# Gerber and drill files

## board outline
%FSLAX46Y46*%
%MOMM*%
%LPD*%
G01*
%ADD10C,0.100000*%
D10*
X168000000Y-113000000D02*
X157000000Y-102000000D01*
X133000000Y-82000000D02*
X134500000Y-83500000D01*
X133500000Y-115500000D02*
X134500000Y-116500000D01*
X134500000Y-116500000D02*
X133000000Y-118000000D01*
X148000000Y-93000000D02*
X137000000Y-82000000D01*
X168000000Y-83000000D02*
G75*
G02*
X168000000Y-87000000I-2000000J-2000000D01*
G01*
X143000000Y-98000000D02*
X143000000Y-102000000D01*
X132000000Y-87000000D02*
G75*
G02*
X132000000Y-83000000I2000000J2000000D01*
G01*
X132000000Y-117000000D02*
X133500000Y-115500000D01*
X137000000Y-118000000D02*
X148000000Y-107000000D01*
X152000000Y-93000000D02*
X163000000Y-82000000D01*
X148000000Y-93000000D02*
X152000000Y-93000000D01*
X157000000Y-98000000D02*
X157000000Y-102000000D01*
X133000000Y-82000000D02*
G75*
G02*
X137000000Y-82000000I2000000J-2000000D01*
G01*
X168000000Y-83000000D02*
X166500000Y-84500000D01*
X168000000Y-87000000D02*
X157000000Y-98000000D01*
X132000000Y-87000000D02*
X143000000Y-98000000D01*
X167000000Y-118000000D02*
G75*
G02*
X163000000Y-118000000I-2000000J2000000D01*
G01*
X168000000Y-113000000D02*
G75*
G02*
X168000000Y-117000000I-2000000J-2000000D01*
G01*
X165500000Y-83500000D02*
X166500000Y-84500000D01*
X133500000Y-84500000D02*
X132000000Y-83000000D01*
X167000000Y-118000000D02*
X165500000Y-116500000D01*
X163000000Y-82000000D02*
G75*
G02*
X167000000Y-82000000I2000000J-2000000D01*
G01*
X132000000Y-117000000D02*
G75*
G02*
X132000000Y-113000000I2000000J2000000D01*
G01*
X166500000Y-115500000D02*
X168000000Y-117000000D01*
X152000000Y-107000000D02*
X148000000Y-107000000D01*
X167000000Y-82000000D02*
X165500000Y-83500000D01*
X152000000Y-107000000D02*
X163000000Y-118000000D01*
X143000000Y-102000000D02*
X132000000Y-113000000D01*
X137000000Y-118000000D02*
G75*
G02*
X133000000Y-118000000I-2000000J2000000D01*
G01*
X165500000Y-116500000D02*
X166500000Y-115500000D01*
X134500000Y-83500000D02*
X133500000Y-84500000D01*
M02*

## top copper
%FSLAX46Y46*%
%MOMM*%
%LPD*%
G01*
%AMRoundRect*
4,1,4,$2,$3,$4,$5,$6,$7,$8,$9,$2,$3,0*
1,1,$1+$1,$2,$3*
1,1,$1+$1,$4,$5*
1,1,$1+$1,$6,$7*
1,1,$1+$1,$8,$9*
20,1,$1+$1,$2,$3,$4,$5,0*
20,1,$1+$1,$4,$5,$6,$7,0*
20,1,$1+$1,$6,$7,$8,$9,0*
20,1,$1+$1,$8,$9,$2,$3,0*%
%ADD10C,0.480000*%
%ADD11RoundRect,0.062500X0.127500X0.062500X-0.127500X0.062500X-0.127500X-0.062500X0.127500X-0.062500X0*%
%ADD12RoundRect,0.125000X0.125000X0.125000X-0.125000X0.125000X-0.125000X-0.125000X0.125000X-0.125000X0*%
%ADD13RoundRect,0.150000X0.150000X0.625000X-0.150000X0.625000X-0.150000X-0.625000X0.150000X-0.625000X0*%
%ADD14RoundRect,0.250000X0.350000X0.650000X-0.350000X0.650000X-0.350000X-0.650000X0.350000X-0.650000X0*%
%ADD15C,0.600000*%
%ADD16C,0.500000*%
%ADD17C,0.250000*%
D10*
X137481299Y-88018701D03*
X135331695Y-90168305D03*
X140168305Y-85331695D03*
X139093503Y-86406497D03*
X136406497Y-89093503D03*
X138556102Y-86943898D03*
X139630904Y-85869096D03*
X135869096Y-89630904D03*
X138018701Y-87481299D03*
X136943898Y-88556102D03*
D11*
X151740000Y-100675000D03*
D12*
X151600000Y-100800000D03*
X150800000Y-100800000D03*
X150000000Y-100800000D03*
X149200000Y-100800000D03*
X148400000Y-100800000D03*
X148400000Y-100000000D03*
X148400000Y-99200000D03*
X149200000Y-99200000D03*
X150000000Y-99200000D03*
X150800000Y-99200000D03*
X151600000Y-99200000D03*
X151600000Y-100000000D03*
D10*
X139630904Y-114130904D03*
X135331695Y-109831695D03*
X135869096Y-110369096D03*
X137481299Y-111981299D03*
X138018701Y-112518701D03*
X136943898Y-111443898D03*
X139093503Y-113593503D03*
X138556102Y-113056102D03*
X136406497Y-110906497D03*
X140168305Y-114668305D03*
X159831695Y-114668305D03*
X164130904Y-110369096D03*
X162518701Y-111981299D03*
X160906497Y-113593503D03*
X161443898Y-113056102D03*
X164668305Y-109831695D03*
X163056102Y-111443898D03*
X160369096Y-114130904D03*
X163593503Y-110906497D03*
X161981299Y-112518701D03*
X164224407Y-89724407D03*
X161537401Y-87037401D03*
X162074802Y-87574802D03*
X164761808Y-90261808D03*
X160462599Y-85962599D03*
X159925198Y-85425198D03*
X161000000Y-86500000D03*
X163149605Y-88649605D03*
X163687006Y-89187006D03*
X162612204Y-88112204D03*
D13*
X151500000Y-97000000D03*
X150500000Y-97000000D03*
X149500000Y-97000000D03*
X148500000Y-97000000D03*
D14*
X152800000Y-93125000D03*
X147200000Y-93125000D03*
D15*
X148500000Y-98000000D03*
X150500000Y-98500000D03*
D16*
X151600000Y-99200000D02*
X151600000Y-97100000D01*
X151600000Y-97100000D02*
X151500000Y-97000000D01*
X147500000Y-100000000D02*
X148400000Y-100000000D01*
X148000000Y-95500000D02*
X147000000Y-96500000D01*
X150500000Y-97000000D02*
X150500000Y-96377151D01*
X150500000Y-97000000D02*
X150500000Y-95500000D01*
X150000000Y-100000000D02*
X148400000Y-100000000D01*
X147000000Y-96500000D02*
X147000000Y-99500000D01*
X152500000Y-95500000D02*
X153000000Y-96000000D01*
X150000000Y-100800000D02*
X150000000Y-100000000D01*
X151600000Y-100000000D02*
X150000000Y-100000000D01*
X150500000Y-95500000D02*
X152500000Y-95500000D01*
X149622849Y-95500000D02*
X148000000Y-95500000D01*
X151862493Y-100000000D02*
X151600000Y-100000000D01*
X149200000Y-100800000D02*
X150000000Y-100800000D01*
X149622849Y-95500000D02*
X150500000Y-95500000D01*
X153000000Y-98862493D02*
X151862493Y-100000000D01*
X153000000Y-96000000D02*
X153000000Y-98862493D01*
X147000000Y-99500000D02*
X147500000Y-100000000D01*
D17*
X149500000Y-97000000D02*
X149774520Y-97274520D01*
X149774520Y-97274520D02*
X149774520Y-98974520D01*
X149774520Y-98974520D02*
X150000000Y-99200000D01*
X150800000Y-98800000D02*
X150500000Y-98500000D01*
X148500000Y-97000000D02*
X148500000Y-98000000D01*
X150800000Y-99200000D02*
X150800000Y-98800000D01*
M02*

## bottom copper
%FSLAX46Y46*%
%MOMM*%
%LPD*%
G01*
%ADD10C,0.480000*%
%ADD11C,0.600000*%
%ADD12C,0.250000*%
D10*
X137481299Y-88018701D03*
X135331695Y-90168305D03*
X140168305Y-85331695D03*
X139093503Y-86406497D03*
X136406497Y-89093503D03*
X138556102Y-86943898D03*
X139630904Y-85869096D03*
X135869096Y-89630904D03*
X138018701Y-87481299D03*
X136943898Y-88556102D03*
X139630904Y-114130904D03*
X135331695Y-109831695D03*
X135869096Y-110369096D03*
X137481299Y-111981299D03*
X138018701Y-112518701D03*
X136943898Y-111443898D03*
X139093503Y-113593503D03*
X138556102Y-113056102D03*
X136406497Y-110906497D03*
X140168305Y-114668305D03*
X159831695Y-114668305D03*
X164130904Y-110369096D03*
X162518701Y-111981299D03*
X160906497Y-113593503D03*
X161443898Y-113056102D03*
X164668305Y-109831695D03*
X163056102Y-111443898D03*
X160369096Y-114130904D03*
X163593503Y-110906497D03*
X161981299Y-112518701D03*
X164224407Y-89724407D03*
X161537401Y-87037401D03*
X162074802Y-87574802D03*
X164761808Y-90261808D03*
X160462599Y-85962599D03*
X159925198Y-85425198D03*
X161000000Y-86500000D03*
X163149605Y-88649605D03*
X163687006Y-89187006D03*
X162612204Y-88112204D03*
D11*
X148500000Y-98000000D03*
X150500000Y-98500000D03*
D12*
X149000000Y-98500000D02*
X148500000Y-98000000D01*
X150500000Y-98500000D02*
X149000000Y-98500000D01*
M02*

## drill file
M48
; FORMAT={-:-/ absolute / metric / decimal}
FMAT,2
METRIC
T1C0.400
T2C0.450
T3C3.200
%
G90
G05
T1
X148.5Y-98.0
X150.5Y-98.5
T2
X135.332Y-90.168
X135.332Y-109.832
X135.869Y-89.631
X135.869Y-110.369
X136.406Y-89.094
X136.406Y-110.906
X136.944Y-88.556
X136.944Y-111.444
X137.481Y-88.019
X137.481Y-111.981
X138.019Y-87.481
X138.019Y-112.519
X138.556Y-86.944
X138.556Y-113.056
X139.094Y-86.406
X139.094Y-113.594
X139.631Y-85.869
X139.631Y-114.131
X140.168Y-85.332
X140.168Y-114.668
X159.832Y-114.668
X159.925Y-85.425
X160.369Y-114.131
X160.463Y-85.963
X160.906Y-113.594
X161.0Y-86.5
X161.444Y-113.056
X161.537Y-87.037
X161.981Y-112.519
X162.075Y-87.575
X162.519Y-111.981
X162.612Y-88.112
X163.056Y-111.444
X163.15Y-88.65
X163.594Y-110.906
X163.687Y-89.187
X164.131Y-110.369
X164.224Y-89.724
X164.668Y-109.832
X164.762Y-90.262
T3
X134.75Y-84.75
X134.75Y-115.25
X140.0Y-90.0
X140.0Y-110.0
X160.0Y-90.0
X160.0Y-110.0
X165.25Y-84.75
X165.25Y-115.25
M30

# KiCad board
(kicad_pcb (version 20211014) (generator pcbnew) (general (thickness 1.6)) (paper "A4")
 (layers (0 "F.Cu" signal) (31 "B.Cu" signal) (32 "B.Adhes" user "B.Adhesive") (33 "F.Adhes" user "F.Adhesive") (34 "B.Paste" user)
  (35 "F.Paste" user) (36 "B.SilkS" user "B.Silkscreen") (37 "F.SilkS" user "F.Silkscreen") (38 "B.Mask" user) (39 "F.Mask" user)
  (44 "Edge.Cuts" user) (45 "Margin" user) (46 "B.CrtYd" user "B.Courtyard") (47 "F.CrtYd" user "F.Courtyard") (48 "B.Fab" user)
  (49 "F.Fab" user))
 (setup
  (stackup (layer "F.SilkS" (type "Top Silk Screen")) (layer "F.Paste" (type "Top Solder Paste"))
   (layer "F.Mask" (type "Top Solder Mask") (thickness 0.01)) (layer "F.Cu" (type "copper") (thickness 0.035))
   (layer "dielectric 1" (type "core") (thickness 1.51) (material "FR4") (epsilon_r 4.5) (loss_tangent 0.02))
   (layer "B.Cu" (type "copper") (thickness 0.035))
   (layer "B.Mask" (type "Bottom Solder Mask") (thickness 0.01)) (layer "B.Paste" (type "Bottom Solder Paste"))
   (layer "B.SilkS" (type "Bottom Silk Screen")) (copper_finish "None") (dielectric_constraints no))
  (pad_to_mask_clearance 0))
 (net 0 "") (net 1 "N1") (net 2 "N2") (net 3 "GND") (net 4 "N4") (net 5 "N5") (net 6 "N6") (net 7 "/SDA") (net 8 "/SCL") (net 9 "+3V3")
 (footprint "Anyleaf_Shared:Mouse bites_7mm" (layer "F.Cu") (at 137.75 87.75 45)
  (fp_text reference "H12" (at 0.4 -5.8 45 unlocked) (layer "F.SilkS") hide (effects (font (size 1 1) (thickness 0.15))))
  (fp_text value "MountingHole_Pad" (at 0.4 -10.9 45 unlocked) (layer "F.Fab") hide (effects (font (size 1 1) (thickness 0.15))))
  (pad "" np_thru_hole circle (at -0.38 0 45) (size 0.48 0.48) (drill 0.45) (layers F&B.Cu *.Mask))
  (pad "" np_thru_hole circle (at -3.42 0 45) (size 0.48 0.48) (drill 0.45) (layers F&B.Cu *.Mask))
  (pad "" np_thru_hole circle (at 3.42 0 45) (size 0.48 0.48) (drill 0.45) (layers F&B.Cu *.Mask))
  (pad "" np_thru_hole circle (at 1.9 0 45) (size 0.48 0.48) (drill 0.45) (layers F&B.Cu *.Mask))
  (pad "" np_thru_hole circle (at -1.9 0 45) (size 0.48 0.48) (drill 0.45) (layers F&B.Cu *.Mask))
  (pad "" np_thru_hole circle (at 1.14 0 45) (size 0.48 0.48) (drill 0.45) (layers F&B.Cu *.Mask))
  (pad "" np_thru_hole circle (at 2.66 0 45) (size 0.48 0.48) (drill 0.45) (layers F&B.Cu *.Mask))
  (pad "" np_thru_hole circle (at -2.66 0 45) (size 0.48 0.48) (drill 0.45) (layers F&B.Cu *.Mask))
  (pad "" np_thru_hole circle (at 0.38 0 45) (size 0.48 0.48) (drill 0.45) (layers F&B.Cu *.Mask))
  (pad "" np_thru_hole circle (at -1.14 0 45) (size 0.48 0.48) (drill 0.45) (layers F&B.Cu *.Mask)))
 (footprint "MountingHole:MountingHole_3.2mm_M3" (layer "F.Cu") (at 134.75 115.25)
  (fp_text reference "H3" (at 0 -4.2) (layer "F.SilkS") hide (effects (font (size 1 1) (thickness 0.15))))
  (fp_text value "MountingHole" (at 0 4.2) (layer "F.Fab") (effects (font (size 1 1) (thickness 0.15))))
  (pad "" np_thru_hole circle locked (at 0 0) (size 3.2 3.2) (drill 3.2) (layers *.Cu *.Mask)))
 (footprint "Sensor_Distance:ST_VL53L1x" (layer "F.Cu") (at 150 100 180)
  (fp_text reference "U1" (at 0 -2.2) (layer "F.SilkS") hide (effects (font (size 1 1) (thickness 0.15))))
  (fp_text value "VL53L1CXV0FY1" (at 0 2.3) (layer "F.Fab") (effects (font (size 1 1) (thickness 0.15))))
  (pad "1" smd roundrect locked (at -1.74 -0.675 180) (size 0.38 0.25) (layers "F.Cu" "F.Paste" "F.Mask") (roundrect_rratio 0.25)
   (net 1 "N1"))
  (pad "1" smd roundrect locked (at -1.6 -0.8 180) (size 0.5 0.5) (layers "F.Cu" "F.Paste" "F.Mask") (roundrect_rratio 0.25) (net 1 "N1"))
  (pad "2" smd roundrect locked (at -0.8 -0.8 180) (size 0.5 0.5) (layers "F.Cu" "F.Paste" "F.Mask") (roundrect_rratio 0.25) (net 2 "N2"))
  (pad "3" smd roundrect locked (at 0 -0.8 180) (size 0.5 0.5) (layers "F.Cu" "F.Paste" "F.Mask") (roundrect_rratio 0.25) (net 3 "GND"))
  (pad "4" smd roundrect locked (at 0.8 -0.8 180) (size 0.5 0.5) (layers "F.Cu" "F.Paste" "F.Mask") (roundrect_rratio 0.25) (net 3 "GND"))
  (pad "5" smd roundrect locked (at 1.6 -0.8 180) (size 0.5 0.5) (layers "F.Cu" "F.Paste" "F.Mask") (roundrect_rratio 0.25) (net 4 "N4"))
  (pad "6" smd roundrect locked (at 1.6 0 180) (size 0.5 0.5) (layers "F.Cu" "F.Paste" "F.Mask") (roundrect_rratio 0.25) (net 3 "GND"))
  (pad "7" smd roundrect locked (at 1.6 0.8 180) (size 0.5 0.5) (layers "F.Cu" "F.Paste" "F.Mask") (roundrect_rratio 0.25) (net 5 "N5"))
  (pad "8" smd roundrect locked (at 0.8 0.8 180) (size 0.5 0.5) (layers "F.Cu" "F.Paste" "F.Mask") (roundrect_rratio 0.25) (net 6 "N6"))
  (pad "9" smd roundrect locked (at 0 0.8 180) (size 0.5 0.5) (layers "F.Cu" "F.Paste" "F.Mask") (roundrect_rratio 0.25) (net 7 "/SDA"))
  (pad "10" smd roundrect locked (at -0.8 0.8 180) (size 0.5 0.5) (layers "F.Cu" "F.Paste" "F.Mask") (roundrect_rratio 0.25) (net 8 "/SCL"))
  (pad "11" smd roundrect locked (at -1.6 0.8 180) (size 0.5 0.5) (layers "F.Cu" "F.Paste" "F.Mask") (roundrect_rratio 0.25) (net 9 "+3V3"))
  (pad "12" smd roundrect locked (at -1.6 0 180) (size 0.5 0.5) (layers "F.Cu" "F.Paste" "F.Mask") (roundrect_rratio 0.25) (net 3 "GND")))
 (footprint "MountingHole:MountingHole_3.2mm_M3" (layer "F.Cu") (at 134.75 84.75)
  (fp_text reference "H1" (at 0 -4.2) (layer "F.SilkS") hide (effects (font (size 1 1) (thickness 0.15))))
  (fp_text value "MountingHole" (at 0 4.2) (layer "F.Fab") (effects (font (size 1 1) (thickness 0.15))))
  (pad "" np_thru_hole circle locked (at 0 0) (size 3.2 3.2) (drill 3.2) (layers *.Cu *.Mask)))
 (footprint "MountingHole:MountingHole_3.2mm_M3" (layer "F.Cu") (at 140 90)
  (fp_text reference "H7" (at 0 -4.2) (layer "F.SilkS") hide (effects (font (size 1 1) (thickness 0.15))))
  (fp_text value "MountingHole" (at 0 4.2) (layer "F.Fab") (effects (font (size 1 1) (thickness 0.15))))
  (pad "" np_thru_hole circle locked (at 0 0) (size 3.2 3.2) (drill 3.2) (layers *.Cu *.Mask)))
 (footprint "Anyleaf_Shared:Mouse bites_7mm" (layer "F.Cu") (at 137.75 112.25 135)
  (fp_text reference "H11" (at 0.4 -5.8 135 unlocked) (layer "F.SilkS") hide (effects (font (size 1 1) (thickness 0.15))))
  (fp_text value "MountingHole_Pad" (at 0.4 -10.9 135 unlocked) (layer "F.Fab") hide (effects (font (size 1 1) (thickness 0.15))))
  (pad "" np_thru_hole circle (at -2.66 0 135) (size 0.48 0.48) (drill 0.45) (layers F&B.Cu *.Mask))
  (pad "" np_thru_hole circle (at 3.42 0 135) (size 0.48 0.48) (drill 0.45) (layers F&B.Cu *.Mask))
  (pad "" np_thru_hole circle (at 2.66 0 135) (size 0.48 0.48) (drill 0.45) (layers F&B.Cu *.Mask))
  (pad "" np_thru_hole circle (at 0.38 0 135) (size 0.48 0.48) (drill 0.45) (layers F&B.Cu *.Mask))
  (pad "" np_thru_hole circle (at -0.38 0 135) (size 0.48 0.48) (drill 0.45) (layers F&B.Cu *.Mask))
  (pad "" np_thru_hole circle (at 1.14 0 135) (size 0.48 0.48) (drill 0.45) (layers F&B.Cu *.Mask))
  (pad "" np_thru_hole circle (at -1.9 0 135) (size 0.48 0.48) (drill 0.45) (layers F&B.Cu *.Mask))
  (pad "" np_thru_hole circle (at -1.14 0 135) (size 0.48 0.48) (drill 0.45) (layers F&B.Cu *.Mask))
  (pad "" np_thru_hole circle (at 1.9 0 135) (size 0.48 0.48) (drill 0.45) (layers F&B.Cu *.Mask))
  (pad "" np_thru_hole circle (at -3.42 0 135) (size 0.48 0.48) (drill 0.45) (layers F&B.Cu *.Mask)))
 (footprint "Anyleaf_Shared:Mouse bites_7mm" (layer "F.Cu") (at 162.25 112.25 45)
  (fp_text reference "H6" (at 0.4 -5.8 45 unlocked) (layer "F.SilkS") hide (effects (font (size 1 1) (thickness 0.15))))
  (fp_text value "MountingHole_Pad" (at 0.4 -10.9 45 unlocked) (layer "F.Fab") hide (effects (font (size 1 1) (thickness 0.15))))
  (pad "" np_thru_hole circle (at -3.42 0 45) (size 0.48 0.48) (drill 0.45) (layers F&B.Cu *.Mask))
  (pad "" np_thru_hole circle (at 2.66 0 45) (size 0.48 0.48) (drill 0.45) (layers F&B.Cu *.Mask))
  (pad "" np_thru_hole circle (at 0.38 0 45) (size 0.48 0.48) (drill 0.45) (layers F&B.Cu *.Mask))
  (pad "" np_thru_hole circle (at -1.9 0 45) (size 0.48 0.48) (drill 0.45) (layers F&B.Cu *.Mask))
  (pad "" np_thru_hole circle (at -1.14 0 45) (size 0.48 0.48) (drill 0.45) (layers F&B.Cu *.Mask))
  (pad "" np_thru_hole circle (at 3.42 0 45) (size 0.48 0.48) (drill 0.45) (layers F&B.Cu *.Mask))
  (pad "" np_thru_hole circle (at 1.14 0 45) (size 0.48 0.48) (drill 0.45) (layers F&B.Cu *.Mask))
  (pad "" np_thru_hole circle (at -2.66 0 45) (size 0.48 0.48) (drill 0.45) (layers F&B.Cu *.Mask))
  (pad "" np_thru_hole circle (at 1.9 0 45) (size 0.48 0.48) (drill 0.45) (layers F&B.Cu *.Mask))
  (pad "" np_thru_hole circle (at -0.38 0 45) (size 0.48 0.48) (drill 0.45) (layers F&B.Cu *.Mask)))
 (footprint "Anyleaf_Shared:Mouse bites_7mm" (layer "F.Cu") (at 162.343503 87.843503 135)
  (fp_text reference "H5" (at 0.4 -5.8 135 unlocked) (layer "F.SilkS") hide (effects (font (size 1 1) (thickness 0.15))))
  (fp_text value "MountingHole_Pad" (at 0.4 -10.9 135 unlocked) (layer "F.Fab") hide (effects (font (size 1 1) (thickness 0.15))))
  (pad "" np_thru_hole circle (at -2.66 0 135) (size 0.48 0.48) (drill 0.45) (layers F&B.Cu *.Mask))
  (pad "" np_thru_hole circle (at 1.14 0 135) (size 0.48 0.48) (drill 0.45) (layers F&B.Cu *.Mask))
  (pad "" np_thru_hole circle (at 0.38 0 135) (size 0.48 0.48) (drill 0.45) (layers F&B.Cu *.Mask))
  (pad "" np_thru_hole circle (at -3.42 0 135) (size 0.48 0.48) (drill 0.45) (layers F&B.Cu *.Mask))
  (pad "" np_thru_hole circle (at 2.66 0 135) (size 0.48 0.48) (drill 0.45) (layers F&B.Cu *.Mask))
  (pad "" np_thru_hole circle (at 3.42 0 135) (size 0.48 0.48) (drill 0.45) (layers F&B.Cu *.Mask))
  (pad "" np_thru_hole circle (at 1.9 0 135) (size 0.48 0.48) (drill 0.45) (layers F&B.Cu *.Mask))
  (pad "" np_thru_hole circle (at -1.14 0 135) (size 0.48 0.48) (drill 0.45) (layers F&B.Cu *.Mask))
  (pad "" np_thru_hole circle (at -1.9 0 135) (size 0.48 0.48) (drill 0.45) (layers F&B.Cu *.Mask))
  (pad "" np_thru_hole circle (at -0.38 0 135) (size 0.48 0.48) (drill 0.45) (layers F&B.Cu *.Mask)))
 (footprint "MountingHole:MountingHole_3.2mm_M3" (layer "F.Cu") (at 160 90)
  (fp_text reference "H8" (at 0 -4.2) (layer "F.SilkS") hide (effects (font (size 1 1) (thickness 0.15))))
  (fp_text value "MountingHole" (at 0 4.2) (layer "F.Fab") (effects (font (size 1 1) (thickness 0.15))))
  (pad "" np_thru_hole circle locked (at 0 0) (size 3.2 3.2) (drill 3.2) (layers *.Cu *.Mask)))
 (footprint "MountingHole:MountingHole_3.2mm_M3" (layer "F.Cu") (at 160 110)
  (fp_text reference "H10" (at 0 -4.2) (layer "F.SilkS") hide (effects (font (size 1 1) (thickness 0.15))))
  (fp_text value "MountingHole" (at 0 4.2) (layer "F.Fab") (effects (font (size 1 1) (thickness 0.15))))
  (pad "" np_thru_hole circle locked (at 0 0) (size 3.2 3.2) (drill 3.2) (layers *.Cu *.Mask)))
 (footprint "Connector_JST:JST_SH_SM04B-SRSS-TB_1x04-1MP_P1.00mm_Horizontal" (layer "F.Cu") (at 150 95 180)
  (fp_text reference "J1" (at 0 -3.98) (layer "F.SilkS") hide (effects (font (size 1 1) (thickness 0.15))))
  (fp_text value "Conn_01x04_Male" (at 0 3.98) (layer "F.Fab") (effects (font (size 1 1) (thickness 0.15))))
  (pad "1" smd roundrect locked (at -1.5 -2 180) (size 0.6 1.55) (layers "F.Cu" "F.Paste" "F.Mask") (roundrect_rratio 0.25) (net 9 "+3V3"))
  (pad "2" smd roundrect locked (at -0.5 -2 180) (size 0.6 1.55) (layers "F.Cu" "F.Paste" "F.Mask") (roundrect_rratio 0.25) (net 3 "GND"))
  (pad "3" smd roundrect locked (at 0.5 -2 180) (size 0.6 1.55) (layers "F.Cu" "F.Paste" "F.Mask") (roundrect_rratio 0.25) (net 7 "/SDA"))
  (pad "4" smd roundrect locked (at 1.5 -2 180) (size 0.6 1.55) (layers "F.Cu" "F.Paste" "F.Mask") (roundrect_rratio 0.25) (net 8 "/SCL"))
  (pad "MP" smd roundrect locked (at -2.8 1.875 180) (size 1.2 1.8) (layers "F.Cu" "F.Paste" "F.Mask") (roundrect_rratio 0.2083333333))
  (pad "MP" smd roundrect locked (at 2.8 1.875 180) (size 1.2 1.8) (layers "F.Cu" "F.Paste" "F.Mask") (roundrect_rratio 0.2083333333)))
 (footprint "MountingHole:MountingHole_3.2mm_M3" (layer "F.Cu") (at 165.25 115.25)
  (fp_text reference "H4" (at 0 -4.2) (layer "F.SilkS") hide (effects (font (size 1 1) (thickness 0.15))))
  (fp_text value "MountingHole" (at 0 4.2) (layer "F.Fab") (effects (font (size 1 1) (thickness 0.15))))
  (pad "" np_thru_hole circle locked (at 0 0) (size 3.2 3.2) (drill 3.2) (layers *.Cu *.Mask)))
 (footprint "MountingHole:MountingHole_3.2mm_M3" (layer "F.Cu") (at 165.25 84.75)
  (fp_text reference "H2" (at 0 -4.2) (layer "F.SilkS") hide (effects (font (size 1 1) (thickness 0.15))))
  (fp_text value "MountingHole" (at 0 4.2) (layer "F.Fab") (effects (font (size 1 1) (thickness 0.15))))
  (pad "" np_thru_hole circle locked (at 0 0) (size 3.2 3.2) (drill 3.2) (layers *.Cu *.Mask)))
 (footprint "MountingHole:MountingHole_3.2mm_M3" (layer "F.Cu") (at 140 110)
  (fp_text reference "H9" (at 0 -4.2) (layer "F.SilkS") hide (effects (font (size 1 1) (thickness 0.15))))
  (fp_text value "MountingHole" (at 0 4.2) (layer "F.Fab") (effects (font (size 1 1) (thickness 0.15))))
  (pad "" np_thru_hole circle locked (at 0 0) (size 3.2 3.2) (drill 3.2) (layers *.Cu *.Mask)))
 (gr_line (start 168 113) (end 157 102) (layer "Edge.Cuts") (width 0.1))
 (gr_line (start 133 82) (end 134.5 83.5) (layer "Edge.Cuts") (width 0.1))
 (gr_line (start 133.5 115.5) (end 134.5 116.5) (layer "Edge.Cuts") (width 0.1))
 (gr_line (start 134.5 116.5) (end 133 118) (layer "Edge.Cuts") (width 0.1))
 (gr_line (start 148 93) (end 137 82) (layer "Edge.Cuts") (width 0.1))
 (gr_arc (start 168 83) (mid 168.828427 85) (end 168 87) (layer "Edge.Cuts") (width 0.1))
 (gr_line (start 143 98) (end 143 102) (layer "Edge.Cuts") (width 0.1))
 (gr_arc (start 132 87) (mid 131.171573 85) (end 132 83) (layer "Edge.Cuts") (width 0.1))
 (gr_line (start 132 117) (end 133.5 115.5) (layer "Edge.Cuts") (width 0.1))
 (gr_line (start 137 118) (end 148 107) (layer "Edge.Cuts") (width 0.1))
 (gr_line (start 152 93) (end 163 82) (layer "Edge.Cuts") (width 0.1))
 (gr_line (start 148 93) (end 152 93) (layer "Edge.Cuts") (width 0.1))
 (gr_line (start 157 98) (end 157 102) (layer "Edge.Cuts") (width 0.1))
 (gr_arc (start 133 82) (mid 135 81.171573) (end 137 82) (layer "Edge.Cuts") (width 0.1))
 (gr_line (start 168 83) (end 166.5 84.5) (layer "Edge.Cuts") (width 0.1))
 (gr_line (start 168 87) (end 157 98) (layer "Edge.Cuts") (width 0.1))
 (gr_line (start 132 87) (end 143 98) (layer "Edge.Cuts") (width 0.1))
 (gr_arc (start 167 118) (mid 165 118.828427) (end 163 118) (layer "Edge.Cuts") (width 0.1))
 (gr_arc (start 168 113) (mid 168.828427 115) (end 168 117) (layer "Edge.Cuts") (width 0.1))
 (gr_line (start 165.5 83.5) (end 166.5 84.5) (layer "Edge.Cuts") (width 0.1))
 (gr_line (start 133.5 84.5) (end 132 83) (layer "Edge.Cuts") (width 0.1))
 (gr_line (start 167 118) (end 165.5 116.5) (layer "Edge.Cuts") (width 0.1))
 (gr_arc (start 163 82) (mid 165 81.171573) (end 167 82) (layer "Edge.Cuts") (width 0.1))
 (gr_arc (start 132 117) (mid 131.171573 115) (end 132 113) (layer "Edge.Cuts") (width 0.1))
 (gr_line (start 166.5 115.5) (end 168 117) (layer "Edge.Cuts") (width 0.1))
 (gr_line (start 152 107) (end 148 107) (layer "Edge.Cuts") (width 0.1))
 (gr_line (start 167 82) (end 165.5 83.5) (layer "Edge.Cuts") (width 0.1))
 (gr_line (start 152 107) (end 163 118) (layer "Edge.Cuts") (width 0.1))
 (gr_line (start 143 102) (end 132 113) (layer "Edge.Cuts") (width 0.1))
 (gr_arc (start 137 118) (mid 135 118.828427) (end 133 118) (layer "Edge.Cuts") (width 0.1))
 (gr_line (start 165.5 116.5) (end 166.5 115.5) (layer "Edge.Cuts") (width 0.1))
 (gr_line (start 134.5 83.5) (end 133.5 84.5) (layer "Edge.Cuts") (width 0.1))
 (segment (start 151.6 99.2) (end 151.6 97.1) (width 0.5) (layer "F.Cu") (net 9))
 (segment (start 151.6 97.1) (end 151.5 97) (width 0.5) (layer "F.Cu") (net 9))
 (segment (start 147.5 100) (end 148.4 100) (width 0.5) (layer "F.Cu") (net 3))
 (segment (start 148 95.5) (end 147 96.5) (width 0.5) (layer "F.Cu") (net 3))
 (segment (start 150.5 97) (end 150.5 96.377151) (width 0.5) (layer "F.Cu") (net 3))
 (segment (start 150.5 97) (end 150.5 95.5) (width 0.5) (layer "F.Cu") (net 3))
 (segment (start 150 100) (end 148.4 100) (width 0.5) (layer "F.Cu") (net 3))
 (segment (start 147 96.5) (end 147 99.5) (width 0.5) (layer "F.Cu") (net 3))
 (segment (start 152.5 95.5) (end 153 96) (width 0.5) (layer "F.Cu") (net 3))
 (segment (start 150 100.8) (end 150 100) (width 0.5) (layer "F.Cu") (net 3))
 (segment (start 151.6 100) (end 150 100) (width 0.5) (layer "F.Cu") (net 3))
 (segment (start 150.5 95.5) (end 152.5 95.5) (width 0.5) (layer "F.Cu") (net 3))
 (segment (start 149.622849 95.5) (end 148 95.5) (width 0.5) (layer "F.Cu") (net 3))
 (segment (start 151.862493 100) (end 151.6 100) (width 0.5) (layer "F.Cu") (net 3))
 (segment (start 149.2 100.8) (end 150 100.8) (width 0.5) (layer "F.Cu") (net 3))
 (segment (start 149.622849 95.5) (end 150.5 95.5) (width 0.5) (layer "F.Cu") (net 3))
 (segment (start 153 98.862493) (end 151.862493 100) (width 0.5) (layer "F.Cu") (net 3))
 (segment (start 153 96) (end 153 98.862493) (width 0.5) (layer "F.Cu") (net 3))
 (segment (start 147 99.5) (end 147.5 100) (width 0.5) (layer "F.Cu") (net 3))
 (segment (start 149.5 97) (end 149.77452 97.27452) (width 0.25) (layer "F.Cu") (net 7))
 (segment (start 149.77452 97.27452) (end 149.77452 98.97452) (width 0.25) (layer "F.Cu") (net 7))
 (segment (start 149.77452 98.97452) (end 150 99.2) (width 0.25) (layer "F.Cu") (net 7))
 (segment (start 150.8 98.8) (end 150.5 98.5) (width 0.25) (layer "F.Cu") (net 8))
 (segment (start 148.5 97) (end 148.5 98) (width 0.25) (layer "F.Cu") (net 8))
 (segment (start 150.8 99.2) (end 150.8 98.8) (width 0.25) (layer "F.Cu") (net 8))
 (via (at 148.5 98) (size 0.6) (drill 0.4) (layers "F.Cu" "B.Cu") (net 8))
 (via (at 150.5 98.5) (size 0.6) (drill 0.4) (layers "F.Cu" "B.Cu") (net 8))
 (segment (start 149 98.5) (end 148.5 98) (width 0.25) (layer "B.Cu") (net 8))
 (segment (start 150.5 98.5) (end 149 98.5) (width 0.25) (layer "B.Cu") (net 8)))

